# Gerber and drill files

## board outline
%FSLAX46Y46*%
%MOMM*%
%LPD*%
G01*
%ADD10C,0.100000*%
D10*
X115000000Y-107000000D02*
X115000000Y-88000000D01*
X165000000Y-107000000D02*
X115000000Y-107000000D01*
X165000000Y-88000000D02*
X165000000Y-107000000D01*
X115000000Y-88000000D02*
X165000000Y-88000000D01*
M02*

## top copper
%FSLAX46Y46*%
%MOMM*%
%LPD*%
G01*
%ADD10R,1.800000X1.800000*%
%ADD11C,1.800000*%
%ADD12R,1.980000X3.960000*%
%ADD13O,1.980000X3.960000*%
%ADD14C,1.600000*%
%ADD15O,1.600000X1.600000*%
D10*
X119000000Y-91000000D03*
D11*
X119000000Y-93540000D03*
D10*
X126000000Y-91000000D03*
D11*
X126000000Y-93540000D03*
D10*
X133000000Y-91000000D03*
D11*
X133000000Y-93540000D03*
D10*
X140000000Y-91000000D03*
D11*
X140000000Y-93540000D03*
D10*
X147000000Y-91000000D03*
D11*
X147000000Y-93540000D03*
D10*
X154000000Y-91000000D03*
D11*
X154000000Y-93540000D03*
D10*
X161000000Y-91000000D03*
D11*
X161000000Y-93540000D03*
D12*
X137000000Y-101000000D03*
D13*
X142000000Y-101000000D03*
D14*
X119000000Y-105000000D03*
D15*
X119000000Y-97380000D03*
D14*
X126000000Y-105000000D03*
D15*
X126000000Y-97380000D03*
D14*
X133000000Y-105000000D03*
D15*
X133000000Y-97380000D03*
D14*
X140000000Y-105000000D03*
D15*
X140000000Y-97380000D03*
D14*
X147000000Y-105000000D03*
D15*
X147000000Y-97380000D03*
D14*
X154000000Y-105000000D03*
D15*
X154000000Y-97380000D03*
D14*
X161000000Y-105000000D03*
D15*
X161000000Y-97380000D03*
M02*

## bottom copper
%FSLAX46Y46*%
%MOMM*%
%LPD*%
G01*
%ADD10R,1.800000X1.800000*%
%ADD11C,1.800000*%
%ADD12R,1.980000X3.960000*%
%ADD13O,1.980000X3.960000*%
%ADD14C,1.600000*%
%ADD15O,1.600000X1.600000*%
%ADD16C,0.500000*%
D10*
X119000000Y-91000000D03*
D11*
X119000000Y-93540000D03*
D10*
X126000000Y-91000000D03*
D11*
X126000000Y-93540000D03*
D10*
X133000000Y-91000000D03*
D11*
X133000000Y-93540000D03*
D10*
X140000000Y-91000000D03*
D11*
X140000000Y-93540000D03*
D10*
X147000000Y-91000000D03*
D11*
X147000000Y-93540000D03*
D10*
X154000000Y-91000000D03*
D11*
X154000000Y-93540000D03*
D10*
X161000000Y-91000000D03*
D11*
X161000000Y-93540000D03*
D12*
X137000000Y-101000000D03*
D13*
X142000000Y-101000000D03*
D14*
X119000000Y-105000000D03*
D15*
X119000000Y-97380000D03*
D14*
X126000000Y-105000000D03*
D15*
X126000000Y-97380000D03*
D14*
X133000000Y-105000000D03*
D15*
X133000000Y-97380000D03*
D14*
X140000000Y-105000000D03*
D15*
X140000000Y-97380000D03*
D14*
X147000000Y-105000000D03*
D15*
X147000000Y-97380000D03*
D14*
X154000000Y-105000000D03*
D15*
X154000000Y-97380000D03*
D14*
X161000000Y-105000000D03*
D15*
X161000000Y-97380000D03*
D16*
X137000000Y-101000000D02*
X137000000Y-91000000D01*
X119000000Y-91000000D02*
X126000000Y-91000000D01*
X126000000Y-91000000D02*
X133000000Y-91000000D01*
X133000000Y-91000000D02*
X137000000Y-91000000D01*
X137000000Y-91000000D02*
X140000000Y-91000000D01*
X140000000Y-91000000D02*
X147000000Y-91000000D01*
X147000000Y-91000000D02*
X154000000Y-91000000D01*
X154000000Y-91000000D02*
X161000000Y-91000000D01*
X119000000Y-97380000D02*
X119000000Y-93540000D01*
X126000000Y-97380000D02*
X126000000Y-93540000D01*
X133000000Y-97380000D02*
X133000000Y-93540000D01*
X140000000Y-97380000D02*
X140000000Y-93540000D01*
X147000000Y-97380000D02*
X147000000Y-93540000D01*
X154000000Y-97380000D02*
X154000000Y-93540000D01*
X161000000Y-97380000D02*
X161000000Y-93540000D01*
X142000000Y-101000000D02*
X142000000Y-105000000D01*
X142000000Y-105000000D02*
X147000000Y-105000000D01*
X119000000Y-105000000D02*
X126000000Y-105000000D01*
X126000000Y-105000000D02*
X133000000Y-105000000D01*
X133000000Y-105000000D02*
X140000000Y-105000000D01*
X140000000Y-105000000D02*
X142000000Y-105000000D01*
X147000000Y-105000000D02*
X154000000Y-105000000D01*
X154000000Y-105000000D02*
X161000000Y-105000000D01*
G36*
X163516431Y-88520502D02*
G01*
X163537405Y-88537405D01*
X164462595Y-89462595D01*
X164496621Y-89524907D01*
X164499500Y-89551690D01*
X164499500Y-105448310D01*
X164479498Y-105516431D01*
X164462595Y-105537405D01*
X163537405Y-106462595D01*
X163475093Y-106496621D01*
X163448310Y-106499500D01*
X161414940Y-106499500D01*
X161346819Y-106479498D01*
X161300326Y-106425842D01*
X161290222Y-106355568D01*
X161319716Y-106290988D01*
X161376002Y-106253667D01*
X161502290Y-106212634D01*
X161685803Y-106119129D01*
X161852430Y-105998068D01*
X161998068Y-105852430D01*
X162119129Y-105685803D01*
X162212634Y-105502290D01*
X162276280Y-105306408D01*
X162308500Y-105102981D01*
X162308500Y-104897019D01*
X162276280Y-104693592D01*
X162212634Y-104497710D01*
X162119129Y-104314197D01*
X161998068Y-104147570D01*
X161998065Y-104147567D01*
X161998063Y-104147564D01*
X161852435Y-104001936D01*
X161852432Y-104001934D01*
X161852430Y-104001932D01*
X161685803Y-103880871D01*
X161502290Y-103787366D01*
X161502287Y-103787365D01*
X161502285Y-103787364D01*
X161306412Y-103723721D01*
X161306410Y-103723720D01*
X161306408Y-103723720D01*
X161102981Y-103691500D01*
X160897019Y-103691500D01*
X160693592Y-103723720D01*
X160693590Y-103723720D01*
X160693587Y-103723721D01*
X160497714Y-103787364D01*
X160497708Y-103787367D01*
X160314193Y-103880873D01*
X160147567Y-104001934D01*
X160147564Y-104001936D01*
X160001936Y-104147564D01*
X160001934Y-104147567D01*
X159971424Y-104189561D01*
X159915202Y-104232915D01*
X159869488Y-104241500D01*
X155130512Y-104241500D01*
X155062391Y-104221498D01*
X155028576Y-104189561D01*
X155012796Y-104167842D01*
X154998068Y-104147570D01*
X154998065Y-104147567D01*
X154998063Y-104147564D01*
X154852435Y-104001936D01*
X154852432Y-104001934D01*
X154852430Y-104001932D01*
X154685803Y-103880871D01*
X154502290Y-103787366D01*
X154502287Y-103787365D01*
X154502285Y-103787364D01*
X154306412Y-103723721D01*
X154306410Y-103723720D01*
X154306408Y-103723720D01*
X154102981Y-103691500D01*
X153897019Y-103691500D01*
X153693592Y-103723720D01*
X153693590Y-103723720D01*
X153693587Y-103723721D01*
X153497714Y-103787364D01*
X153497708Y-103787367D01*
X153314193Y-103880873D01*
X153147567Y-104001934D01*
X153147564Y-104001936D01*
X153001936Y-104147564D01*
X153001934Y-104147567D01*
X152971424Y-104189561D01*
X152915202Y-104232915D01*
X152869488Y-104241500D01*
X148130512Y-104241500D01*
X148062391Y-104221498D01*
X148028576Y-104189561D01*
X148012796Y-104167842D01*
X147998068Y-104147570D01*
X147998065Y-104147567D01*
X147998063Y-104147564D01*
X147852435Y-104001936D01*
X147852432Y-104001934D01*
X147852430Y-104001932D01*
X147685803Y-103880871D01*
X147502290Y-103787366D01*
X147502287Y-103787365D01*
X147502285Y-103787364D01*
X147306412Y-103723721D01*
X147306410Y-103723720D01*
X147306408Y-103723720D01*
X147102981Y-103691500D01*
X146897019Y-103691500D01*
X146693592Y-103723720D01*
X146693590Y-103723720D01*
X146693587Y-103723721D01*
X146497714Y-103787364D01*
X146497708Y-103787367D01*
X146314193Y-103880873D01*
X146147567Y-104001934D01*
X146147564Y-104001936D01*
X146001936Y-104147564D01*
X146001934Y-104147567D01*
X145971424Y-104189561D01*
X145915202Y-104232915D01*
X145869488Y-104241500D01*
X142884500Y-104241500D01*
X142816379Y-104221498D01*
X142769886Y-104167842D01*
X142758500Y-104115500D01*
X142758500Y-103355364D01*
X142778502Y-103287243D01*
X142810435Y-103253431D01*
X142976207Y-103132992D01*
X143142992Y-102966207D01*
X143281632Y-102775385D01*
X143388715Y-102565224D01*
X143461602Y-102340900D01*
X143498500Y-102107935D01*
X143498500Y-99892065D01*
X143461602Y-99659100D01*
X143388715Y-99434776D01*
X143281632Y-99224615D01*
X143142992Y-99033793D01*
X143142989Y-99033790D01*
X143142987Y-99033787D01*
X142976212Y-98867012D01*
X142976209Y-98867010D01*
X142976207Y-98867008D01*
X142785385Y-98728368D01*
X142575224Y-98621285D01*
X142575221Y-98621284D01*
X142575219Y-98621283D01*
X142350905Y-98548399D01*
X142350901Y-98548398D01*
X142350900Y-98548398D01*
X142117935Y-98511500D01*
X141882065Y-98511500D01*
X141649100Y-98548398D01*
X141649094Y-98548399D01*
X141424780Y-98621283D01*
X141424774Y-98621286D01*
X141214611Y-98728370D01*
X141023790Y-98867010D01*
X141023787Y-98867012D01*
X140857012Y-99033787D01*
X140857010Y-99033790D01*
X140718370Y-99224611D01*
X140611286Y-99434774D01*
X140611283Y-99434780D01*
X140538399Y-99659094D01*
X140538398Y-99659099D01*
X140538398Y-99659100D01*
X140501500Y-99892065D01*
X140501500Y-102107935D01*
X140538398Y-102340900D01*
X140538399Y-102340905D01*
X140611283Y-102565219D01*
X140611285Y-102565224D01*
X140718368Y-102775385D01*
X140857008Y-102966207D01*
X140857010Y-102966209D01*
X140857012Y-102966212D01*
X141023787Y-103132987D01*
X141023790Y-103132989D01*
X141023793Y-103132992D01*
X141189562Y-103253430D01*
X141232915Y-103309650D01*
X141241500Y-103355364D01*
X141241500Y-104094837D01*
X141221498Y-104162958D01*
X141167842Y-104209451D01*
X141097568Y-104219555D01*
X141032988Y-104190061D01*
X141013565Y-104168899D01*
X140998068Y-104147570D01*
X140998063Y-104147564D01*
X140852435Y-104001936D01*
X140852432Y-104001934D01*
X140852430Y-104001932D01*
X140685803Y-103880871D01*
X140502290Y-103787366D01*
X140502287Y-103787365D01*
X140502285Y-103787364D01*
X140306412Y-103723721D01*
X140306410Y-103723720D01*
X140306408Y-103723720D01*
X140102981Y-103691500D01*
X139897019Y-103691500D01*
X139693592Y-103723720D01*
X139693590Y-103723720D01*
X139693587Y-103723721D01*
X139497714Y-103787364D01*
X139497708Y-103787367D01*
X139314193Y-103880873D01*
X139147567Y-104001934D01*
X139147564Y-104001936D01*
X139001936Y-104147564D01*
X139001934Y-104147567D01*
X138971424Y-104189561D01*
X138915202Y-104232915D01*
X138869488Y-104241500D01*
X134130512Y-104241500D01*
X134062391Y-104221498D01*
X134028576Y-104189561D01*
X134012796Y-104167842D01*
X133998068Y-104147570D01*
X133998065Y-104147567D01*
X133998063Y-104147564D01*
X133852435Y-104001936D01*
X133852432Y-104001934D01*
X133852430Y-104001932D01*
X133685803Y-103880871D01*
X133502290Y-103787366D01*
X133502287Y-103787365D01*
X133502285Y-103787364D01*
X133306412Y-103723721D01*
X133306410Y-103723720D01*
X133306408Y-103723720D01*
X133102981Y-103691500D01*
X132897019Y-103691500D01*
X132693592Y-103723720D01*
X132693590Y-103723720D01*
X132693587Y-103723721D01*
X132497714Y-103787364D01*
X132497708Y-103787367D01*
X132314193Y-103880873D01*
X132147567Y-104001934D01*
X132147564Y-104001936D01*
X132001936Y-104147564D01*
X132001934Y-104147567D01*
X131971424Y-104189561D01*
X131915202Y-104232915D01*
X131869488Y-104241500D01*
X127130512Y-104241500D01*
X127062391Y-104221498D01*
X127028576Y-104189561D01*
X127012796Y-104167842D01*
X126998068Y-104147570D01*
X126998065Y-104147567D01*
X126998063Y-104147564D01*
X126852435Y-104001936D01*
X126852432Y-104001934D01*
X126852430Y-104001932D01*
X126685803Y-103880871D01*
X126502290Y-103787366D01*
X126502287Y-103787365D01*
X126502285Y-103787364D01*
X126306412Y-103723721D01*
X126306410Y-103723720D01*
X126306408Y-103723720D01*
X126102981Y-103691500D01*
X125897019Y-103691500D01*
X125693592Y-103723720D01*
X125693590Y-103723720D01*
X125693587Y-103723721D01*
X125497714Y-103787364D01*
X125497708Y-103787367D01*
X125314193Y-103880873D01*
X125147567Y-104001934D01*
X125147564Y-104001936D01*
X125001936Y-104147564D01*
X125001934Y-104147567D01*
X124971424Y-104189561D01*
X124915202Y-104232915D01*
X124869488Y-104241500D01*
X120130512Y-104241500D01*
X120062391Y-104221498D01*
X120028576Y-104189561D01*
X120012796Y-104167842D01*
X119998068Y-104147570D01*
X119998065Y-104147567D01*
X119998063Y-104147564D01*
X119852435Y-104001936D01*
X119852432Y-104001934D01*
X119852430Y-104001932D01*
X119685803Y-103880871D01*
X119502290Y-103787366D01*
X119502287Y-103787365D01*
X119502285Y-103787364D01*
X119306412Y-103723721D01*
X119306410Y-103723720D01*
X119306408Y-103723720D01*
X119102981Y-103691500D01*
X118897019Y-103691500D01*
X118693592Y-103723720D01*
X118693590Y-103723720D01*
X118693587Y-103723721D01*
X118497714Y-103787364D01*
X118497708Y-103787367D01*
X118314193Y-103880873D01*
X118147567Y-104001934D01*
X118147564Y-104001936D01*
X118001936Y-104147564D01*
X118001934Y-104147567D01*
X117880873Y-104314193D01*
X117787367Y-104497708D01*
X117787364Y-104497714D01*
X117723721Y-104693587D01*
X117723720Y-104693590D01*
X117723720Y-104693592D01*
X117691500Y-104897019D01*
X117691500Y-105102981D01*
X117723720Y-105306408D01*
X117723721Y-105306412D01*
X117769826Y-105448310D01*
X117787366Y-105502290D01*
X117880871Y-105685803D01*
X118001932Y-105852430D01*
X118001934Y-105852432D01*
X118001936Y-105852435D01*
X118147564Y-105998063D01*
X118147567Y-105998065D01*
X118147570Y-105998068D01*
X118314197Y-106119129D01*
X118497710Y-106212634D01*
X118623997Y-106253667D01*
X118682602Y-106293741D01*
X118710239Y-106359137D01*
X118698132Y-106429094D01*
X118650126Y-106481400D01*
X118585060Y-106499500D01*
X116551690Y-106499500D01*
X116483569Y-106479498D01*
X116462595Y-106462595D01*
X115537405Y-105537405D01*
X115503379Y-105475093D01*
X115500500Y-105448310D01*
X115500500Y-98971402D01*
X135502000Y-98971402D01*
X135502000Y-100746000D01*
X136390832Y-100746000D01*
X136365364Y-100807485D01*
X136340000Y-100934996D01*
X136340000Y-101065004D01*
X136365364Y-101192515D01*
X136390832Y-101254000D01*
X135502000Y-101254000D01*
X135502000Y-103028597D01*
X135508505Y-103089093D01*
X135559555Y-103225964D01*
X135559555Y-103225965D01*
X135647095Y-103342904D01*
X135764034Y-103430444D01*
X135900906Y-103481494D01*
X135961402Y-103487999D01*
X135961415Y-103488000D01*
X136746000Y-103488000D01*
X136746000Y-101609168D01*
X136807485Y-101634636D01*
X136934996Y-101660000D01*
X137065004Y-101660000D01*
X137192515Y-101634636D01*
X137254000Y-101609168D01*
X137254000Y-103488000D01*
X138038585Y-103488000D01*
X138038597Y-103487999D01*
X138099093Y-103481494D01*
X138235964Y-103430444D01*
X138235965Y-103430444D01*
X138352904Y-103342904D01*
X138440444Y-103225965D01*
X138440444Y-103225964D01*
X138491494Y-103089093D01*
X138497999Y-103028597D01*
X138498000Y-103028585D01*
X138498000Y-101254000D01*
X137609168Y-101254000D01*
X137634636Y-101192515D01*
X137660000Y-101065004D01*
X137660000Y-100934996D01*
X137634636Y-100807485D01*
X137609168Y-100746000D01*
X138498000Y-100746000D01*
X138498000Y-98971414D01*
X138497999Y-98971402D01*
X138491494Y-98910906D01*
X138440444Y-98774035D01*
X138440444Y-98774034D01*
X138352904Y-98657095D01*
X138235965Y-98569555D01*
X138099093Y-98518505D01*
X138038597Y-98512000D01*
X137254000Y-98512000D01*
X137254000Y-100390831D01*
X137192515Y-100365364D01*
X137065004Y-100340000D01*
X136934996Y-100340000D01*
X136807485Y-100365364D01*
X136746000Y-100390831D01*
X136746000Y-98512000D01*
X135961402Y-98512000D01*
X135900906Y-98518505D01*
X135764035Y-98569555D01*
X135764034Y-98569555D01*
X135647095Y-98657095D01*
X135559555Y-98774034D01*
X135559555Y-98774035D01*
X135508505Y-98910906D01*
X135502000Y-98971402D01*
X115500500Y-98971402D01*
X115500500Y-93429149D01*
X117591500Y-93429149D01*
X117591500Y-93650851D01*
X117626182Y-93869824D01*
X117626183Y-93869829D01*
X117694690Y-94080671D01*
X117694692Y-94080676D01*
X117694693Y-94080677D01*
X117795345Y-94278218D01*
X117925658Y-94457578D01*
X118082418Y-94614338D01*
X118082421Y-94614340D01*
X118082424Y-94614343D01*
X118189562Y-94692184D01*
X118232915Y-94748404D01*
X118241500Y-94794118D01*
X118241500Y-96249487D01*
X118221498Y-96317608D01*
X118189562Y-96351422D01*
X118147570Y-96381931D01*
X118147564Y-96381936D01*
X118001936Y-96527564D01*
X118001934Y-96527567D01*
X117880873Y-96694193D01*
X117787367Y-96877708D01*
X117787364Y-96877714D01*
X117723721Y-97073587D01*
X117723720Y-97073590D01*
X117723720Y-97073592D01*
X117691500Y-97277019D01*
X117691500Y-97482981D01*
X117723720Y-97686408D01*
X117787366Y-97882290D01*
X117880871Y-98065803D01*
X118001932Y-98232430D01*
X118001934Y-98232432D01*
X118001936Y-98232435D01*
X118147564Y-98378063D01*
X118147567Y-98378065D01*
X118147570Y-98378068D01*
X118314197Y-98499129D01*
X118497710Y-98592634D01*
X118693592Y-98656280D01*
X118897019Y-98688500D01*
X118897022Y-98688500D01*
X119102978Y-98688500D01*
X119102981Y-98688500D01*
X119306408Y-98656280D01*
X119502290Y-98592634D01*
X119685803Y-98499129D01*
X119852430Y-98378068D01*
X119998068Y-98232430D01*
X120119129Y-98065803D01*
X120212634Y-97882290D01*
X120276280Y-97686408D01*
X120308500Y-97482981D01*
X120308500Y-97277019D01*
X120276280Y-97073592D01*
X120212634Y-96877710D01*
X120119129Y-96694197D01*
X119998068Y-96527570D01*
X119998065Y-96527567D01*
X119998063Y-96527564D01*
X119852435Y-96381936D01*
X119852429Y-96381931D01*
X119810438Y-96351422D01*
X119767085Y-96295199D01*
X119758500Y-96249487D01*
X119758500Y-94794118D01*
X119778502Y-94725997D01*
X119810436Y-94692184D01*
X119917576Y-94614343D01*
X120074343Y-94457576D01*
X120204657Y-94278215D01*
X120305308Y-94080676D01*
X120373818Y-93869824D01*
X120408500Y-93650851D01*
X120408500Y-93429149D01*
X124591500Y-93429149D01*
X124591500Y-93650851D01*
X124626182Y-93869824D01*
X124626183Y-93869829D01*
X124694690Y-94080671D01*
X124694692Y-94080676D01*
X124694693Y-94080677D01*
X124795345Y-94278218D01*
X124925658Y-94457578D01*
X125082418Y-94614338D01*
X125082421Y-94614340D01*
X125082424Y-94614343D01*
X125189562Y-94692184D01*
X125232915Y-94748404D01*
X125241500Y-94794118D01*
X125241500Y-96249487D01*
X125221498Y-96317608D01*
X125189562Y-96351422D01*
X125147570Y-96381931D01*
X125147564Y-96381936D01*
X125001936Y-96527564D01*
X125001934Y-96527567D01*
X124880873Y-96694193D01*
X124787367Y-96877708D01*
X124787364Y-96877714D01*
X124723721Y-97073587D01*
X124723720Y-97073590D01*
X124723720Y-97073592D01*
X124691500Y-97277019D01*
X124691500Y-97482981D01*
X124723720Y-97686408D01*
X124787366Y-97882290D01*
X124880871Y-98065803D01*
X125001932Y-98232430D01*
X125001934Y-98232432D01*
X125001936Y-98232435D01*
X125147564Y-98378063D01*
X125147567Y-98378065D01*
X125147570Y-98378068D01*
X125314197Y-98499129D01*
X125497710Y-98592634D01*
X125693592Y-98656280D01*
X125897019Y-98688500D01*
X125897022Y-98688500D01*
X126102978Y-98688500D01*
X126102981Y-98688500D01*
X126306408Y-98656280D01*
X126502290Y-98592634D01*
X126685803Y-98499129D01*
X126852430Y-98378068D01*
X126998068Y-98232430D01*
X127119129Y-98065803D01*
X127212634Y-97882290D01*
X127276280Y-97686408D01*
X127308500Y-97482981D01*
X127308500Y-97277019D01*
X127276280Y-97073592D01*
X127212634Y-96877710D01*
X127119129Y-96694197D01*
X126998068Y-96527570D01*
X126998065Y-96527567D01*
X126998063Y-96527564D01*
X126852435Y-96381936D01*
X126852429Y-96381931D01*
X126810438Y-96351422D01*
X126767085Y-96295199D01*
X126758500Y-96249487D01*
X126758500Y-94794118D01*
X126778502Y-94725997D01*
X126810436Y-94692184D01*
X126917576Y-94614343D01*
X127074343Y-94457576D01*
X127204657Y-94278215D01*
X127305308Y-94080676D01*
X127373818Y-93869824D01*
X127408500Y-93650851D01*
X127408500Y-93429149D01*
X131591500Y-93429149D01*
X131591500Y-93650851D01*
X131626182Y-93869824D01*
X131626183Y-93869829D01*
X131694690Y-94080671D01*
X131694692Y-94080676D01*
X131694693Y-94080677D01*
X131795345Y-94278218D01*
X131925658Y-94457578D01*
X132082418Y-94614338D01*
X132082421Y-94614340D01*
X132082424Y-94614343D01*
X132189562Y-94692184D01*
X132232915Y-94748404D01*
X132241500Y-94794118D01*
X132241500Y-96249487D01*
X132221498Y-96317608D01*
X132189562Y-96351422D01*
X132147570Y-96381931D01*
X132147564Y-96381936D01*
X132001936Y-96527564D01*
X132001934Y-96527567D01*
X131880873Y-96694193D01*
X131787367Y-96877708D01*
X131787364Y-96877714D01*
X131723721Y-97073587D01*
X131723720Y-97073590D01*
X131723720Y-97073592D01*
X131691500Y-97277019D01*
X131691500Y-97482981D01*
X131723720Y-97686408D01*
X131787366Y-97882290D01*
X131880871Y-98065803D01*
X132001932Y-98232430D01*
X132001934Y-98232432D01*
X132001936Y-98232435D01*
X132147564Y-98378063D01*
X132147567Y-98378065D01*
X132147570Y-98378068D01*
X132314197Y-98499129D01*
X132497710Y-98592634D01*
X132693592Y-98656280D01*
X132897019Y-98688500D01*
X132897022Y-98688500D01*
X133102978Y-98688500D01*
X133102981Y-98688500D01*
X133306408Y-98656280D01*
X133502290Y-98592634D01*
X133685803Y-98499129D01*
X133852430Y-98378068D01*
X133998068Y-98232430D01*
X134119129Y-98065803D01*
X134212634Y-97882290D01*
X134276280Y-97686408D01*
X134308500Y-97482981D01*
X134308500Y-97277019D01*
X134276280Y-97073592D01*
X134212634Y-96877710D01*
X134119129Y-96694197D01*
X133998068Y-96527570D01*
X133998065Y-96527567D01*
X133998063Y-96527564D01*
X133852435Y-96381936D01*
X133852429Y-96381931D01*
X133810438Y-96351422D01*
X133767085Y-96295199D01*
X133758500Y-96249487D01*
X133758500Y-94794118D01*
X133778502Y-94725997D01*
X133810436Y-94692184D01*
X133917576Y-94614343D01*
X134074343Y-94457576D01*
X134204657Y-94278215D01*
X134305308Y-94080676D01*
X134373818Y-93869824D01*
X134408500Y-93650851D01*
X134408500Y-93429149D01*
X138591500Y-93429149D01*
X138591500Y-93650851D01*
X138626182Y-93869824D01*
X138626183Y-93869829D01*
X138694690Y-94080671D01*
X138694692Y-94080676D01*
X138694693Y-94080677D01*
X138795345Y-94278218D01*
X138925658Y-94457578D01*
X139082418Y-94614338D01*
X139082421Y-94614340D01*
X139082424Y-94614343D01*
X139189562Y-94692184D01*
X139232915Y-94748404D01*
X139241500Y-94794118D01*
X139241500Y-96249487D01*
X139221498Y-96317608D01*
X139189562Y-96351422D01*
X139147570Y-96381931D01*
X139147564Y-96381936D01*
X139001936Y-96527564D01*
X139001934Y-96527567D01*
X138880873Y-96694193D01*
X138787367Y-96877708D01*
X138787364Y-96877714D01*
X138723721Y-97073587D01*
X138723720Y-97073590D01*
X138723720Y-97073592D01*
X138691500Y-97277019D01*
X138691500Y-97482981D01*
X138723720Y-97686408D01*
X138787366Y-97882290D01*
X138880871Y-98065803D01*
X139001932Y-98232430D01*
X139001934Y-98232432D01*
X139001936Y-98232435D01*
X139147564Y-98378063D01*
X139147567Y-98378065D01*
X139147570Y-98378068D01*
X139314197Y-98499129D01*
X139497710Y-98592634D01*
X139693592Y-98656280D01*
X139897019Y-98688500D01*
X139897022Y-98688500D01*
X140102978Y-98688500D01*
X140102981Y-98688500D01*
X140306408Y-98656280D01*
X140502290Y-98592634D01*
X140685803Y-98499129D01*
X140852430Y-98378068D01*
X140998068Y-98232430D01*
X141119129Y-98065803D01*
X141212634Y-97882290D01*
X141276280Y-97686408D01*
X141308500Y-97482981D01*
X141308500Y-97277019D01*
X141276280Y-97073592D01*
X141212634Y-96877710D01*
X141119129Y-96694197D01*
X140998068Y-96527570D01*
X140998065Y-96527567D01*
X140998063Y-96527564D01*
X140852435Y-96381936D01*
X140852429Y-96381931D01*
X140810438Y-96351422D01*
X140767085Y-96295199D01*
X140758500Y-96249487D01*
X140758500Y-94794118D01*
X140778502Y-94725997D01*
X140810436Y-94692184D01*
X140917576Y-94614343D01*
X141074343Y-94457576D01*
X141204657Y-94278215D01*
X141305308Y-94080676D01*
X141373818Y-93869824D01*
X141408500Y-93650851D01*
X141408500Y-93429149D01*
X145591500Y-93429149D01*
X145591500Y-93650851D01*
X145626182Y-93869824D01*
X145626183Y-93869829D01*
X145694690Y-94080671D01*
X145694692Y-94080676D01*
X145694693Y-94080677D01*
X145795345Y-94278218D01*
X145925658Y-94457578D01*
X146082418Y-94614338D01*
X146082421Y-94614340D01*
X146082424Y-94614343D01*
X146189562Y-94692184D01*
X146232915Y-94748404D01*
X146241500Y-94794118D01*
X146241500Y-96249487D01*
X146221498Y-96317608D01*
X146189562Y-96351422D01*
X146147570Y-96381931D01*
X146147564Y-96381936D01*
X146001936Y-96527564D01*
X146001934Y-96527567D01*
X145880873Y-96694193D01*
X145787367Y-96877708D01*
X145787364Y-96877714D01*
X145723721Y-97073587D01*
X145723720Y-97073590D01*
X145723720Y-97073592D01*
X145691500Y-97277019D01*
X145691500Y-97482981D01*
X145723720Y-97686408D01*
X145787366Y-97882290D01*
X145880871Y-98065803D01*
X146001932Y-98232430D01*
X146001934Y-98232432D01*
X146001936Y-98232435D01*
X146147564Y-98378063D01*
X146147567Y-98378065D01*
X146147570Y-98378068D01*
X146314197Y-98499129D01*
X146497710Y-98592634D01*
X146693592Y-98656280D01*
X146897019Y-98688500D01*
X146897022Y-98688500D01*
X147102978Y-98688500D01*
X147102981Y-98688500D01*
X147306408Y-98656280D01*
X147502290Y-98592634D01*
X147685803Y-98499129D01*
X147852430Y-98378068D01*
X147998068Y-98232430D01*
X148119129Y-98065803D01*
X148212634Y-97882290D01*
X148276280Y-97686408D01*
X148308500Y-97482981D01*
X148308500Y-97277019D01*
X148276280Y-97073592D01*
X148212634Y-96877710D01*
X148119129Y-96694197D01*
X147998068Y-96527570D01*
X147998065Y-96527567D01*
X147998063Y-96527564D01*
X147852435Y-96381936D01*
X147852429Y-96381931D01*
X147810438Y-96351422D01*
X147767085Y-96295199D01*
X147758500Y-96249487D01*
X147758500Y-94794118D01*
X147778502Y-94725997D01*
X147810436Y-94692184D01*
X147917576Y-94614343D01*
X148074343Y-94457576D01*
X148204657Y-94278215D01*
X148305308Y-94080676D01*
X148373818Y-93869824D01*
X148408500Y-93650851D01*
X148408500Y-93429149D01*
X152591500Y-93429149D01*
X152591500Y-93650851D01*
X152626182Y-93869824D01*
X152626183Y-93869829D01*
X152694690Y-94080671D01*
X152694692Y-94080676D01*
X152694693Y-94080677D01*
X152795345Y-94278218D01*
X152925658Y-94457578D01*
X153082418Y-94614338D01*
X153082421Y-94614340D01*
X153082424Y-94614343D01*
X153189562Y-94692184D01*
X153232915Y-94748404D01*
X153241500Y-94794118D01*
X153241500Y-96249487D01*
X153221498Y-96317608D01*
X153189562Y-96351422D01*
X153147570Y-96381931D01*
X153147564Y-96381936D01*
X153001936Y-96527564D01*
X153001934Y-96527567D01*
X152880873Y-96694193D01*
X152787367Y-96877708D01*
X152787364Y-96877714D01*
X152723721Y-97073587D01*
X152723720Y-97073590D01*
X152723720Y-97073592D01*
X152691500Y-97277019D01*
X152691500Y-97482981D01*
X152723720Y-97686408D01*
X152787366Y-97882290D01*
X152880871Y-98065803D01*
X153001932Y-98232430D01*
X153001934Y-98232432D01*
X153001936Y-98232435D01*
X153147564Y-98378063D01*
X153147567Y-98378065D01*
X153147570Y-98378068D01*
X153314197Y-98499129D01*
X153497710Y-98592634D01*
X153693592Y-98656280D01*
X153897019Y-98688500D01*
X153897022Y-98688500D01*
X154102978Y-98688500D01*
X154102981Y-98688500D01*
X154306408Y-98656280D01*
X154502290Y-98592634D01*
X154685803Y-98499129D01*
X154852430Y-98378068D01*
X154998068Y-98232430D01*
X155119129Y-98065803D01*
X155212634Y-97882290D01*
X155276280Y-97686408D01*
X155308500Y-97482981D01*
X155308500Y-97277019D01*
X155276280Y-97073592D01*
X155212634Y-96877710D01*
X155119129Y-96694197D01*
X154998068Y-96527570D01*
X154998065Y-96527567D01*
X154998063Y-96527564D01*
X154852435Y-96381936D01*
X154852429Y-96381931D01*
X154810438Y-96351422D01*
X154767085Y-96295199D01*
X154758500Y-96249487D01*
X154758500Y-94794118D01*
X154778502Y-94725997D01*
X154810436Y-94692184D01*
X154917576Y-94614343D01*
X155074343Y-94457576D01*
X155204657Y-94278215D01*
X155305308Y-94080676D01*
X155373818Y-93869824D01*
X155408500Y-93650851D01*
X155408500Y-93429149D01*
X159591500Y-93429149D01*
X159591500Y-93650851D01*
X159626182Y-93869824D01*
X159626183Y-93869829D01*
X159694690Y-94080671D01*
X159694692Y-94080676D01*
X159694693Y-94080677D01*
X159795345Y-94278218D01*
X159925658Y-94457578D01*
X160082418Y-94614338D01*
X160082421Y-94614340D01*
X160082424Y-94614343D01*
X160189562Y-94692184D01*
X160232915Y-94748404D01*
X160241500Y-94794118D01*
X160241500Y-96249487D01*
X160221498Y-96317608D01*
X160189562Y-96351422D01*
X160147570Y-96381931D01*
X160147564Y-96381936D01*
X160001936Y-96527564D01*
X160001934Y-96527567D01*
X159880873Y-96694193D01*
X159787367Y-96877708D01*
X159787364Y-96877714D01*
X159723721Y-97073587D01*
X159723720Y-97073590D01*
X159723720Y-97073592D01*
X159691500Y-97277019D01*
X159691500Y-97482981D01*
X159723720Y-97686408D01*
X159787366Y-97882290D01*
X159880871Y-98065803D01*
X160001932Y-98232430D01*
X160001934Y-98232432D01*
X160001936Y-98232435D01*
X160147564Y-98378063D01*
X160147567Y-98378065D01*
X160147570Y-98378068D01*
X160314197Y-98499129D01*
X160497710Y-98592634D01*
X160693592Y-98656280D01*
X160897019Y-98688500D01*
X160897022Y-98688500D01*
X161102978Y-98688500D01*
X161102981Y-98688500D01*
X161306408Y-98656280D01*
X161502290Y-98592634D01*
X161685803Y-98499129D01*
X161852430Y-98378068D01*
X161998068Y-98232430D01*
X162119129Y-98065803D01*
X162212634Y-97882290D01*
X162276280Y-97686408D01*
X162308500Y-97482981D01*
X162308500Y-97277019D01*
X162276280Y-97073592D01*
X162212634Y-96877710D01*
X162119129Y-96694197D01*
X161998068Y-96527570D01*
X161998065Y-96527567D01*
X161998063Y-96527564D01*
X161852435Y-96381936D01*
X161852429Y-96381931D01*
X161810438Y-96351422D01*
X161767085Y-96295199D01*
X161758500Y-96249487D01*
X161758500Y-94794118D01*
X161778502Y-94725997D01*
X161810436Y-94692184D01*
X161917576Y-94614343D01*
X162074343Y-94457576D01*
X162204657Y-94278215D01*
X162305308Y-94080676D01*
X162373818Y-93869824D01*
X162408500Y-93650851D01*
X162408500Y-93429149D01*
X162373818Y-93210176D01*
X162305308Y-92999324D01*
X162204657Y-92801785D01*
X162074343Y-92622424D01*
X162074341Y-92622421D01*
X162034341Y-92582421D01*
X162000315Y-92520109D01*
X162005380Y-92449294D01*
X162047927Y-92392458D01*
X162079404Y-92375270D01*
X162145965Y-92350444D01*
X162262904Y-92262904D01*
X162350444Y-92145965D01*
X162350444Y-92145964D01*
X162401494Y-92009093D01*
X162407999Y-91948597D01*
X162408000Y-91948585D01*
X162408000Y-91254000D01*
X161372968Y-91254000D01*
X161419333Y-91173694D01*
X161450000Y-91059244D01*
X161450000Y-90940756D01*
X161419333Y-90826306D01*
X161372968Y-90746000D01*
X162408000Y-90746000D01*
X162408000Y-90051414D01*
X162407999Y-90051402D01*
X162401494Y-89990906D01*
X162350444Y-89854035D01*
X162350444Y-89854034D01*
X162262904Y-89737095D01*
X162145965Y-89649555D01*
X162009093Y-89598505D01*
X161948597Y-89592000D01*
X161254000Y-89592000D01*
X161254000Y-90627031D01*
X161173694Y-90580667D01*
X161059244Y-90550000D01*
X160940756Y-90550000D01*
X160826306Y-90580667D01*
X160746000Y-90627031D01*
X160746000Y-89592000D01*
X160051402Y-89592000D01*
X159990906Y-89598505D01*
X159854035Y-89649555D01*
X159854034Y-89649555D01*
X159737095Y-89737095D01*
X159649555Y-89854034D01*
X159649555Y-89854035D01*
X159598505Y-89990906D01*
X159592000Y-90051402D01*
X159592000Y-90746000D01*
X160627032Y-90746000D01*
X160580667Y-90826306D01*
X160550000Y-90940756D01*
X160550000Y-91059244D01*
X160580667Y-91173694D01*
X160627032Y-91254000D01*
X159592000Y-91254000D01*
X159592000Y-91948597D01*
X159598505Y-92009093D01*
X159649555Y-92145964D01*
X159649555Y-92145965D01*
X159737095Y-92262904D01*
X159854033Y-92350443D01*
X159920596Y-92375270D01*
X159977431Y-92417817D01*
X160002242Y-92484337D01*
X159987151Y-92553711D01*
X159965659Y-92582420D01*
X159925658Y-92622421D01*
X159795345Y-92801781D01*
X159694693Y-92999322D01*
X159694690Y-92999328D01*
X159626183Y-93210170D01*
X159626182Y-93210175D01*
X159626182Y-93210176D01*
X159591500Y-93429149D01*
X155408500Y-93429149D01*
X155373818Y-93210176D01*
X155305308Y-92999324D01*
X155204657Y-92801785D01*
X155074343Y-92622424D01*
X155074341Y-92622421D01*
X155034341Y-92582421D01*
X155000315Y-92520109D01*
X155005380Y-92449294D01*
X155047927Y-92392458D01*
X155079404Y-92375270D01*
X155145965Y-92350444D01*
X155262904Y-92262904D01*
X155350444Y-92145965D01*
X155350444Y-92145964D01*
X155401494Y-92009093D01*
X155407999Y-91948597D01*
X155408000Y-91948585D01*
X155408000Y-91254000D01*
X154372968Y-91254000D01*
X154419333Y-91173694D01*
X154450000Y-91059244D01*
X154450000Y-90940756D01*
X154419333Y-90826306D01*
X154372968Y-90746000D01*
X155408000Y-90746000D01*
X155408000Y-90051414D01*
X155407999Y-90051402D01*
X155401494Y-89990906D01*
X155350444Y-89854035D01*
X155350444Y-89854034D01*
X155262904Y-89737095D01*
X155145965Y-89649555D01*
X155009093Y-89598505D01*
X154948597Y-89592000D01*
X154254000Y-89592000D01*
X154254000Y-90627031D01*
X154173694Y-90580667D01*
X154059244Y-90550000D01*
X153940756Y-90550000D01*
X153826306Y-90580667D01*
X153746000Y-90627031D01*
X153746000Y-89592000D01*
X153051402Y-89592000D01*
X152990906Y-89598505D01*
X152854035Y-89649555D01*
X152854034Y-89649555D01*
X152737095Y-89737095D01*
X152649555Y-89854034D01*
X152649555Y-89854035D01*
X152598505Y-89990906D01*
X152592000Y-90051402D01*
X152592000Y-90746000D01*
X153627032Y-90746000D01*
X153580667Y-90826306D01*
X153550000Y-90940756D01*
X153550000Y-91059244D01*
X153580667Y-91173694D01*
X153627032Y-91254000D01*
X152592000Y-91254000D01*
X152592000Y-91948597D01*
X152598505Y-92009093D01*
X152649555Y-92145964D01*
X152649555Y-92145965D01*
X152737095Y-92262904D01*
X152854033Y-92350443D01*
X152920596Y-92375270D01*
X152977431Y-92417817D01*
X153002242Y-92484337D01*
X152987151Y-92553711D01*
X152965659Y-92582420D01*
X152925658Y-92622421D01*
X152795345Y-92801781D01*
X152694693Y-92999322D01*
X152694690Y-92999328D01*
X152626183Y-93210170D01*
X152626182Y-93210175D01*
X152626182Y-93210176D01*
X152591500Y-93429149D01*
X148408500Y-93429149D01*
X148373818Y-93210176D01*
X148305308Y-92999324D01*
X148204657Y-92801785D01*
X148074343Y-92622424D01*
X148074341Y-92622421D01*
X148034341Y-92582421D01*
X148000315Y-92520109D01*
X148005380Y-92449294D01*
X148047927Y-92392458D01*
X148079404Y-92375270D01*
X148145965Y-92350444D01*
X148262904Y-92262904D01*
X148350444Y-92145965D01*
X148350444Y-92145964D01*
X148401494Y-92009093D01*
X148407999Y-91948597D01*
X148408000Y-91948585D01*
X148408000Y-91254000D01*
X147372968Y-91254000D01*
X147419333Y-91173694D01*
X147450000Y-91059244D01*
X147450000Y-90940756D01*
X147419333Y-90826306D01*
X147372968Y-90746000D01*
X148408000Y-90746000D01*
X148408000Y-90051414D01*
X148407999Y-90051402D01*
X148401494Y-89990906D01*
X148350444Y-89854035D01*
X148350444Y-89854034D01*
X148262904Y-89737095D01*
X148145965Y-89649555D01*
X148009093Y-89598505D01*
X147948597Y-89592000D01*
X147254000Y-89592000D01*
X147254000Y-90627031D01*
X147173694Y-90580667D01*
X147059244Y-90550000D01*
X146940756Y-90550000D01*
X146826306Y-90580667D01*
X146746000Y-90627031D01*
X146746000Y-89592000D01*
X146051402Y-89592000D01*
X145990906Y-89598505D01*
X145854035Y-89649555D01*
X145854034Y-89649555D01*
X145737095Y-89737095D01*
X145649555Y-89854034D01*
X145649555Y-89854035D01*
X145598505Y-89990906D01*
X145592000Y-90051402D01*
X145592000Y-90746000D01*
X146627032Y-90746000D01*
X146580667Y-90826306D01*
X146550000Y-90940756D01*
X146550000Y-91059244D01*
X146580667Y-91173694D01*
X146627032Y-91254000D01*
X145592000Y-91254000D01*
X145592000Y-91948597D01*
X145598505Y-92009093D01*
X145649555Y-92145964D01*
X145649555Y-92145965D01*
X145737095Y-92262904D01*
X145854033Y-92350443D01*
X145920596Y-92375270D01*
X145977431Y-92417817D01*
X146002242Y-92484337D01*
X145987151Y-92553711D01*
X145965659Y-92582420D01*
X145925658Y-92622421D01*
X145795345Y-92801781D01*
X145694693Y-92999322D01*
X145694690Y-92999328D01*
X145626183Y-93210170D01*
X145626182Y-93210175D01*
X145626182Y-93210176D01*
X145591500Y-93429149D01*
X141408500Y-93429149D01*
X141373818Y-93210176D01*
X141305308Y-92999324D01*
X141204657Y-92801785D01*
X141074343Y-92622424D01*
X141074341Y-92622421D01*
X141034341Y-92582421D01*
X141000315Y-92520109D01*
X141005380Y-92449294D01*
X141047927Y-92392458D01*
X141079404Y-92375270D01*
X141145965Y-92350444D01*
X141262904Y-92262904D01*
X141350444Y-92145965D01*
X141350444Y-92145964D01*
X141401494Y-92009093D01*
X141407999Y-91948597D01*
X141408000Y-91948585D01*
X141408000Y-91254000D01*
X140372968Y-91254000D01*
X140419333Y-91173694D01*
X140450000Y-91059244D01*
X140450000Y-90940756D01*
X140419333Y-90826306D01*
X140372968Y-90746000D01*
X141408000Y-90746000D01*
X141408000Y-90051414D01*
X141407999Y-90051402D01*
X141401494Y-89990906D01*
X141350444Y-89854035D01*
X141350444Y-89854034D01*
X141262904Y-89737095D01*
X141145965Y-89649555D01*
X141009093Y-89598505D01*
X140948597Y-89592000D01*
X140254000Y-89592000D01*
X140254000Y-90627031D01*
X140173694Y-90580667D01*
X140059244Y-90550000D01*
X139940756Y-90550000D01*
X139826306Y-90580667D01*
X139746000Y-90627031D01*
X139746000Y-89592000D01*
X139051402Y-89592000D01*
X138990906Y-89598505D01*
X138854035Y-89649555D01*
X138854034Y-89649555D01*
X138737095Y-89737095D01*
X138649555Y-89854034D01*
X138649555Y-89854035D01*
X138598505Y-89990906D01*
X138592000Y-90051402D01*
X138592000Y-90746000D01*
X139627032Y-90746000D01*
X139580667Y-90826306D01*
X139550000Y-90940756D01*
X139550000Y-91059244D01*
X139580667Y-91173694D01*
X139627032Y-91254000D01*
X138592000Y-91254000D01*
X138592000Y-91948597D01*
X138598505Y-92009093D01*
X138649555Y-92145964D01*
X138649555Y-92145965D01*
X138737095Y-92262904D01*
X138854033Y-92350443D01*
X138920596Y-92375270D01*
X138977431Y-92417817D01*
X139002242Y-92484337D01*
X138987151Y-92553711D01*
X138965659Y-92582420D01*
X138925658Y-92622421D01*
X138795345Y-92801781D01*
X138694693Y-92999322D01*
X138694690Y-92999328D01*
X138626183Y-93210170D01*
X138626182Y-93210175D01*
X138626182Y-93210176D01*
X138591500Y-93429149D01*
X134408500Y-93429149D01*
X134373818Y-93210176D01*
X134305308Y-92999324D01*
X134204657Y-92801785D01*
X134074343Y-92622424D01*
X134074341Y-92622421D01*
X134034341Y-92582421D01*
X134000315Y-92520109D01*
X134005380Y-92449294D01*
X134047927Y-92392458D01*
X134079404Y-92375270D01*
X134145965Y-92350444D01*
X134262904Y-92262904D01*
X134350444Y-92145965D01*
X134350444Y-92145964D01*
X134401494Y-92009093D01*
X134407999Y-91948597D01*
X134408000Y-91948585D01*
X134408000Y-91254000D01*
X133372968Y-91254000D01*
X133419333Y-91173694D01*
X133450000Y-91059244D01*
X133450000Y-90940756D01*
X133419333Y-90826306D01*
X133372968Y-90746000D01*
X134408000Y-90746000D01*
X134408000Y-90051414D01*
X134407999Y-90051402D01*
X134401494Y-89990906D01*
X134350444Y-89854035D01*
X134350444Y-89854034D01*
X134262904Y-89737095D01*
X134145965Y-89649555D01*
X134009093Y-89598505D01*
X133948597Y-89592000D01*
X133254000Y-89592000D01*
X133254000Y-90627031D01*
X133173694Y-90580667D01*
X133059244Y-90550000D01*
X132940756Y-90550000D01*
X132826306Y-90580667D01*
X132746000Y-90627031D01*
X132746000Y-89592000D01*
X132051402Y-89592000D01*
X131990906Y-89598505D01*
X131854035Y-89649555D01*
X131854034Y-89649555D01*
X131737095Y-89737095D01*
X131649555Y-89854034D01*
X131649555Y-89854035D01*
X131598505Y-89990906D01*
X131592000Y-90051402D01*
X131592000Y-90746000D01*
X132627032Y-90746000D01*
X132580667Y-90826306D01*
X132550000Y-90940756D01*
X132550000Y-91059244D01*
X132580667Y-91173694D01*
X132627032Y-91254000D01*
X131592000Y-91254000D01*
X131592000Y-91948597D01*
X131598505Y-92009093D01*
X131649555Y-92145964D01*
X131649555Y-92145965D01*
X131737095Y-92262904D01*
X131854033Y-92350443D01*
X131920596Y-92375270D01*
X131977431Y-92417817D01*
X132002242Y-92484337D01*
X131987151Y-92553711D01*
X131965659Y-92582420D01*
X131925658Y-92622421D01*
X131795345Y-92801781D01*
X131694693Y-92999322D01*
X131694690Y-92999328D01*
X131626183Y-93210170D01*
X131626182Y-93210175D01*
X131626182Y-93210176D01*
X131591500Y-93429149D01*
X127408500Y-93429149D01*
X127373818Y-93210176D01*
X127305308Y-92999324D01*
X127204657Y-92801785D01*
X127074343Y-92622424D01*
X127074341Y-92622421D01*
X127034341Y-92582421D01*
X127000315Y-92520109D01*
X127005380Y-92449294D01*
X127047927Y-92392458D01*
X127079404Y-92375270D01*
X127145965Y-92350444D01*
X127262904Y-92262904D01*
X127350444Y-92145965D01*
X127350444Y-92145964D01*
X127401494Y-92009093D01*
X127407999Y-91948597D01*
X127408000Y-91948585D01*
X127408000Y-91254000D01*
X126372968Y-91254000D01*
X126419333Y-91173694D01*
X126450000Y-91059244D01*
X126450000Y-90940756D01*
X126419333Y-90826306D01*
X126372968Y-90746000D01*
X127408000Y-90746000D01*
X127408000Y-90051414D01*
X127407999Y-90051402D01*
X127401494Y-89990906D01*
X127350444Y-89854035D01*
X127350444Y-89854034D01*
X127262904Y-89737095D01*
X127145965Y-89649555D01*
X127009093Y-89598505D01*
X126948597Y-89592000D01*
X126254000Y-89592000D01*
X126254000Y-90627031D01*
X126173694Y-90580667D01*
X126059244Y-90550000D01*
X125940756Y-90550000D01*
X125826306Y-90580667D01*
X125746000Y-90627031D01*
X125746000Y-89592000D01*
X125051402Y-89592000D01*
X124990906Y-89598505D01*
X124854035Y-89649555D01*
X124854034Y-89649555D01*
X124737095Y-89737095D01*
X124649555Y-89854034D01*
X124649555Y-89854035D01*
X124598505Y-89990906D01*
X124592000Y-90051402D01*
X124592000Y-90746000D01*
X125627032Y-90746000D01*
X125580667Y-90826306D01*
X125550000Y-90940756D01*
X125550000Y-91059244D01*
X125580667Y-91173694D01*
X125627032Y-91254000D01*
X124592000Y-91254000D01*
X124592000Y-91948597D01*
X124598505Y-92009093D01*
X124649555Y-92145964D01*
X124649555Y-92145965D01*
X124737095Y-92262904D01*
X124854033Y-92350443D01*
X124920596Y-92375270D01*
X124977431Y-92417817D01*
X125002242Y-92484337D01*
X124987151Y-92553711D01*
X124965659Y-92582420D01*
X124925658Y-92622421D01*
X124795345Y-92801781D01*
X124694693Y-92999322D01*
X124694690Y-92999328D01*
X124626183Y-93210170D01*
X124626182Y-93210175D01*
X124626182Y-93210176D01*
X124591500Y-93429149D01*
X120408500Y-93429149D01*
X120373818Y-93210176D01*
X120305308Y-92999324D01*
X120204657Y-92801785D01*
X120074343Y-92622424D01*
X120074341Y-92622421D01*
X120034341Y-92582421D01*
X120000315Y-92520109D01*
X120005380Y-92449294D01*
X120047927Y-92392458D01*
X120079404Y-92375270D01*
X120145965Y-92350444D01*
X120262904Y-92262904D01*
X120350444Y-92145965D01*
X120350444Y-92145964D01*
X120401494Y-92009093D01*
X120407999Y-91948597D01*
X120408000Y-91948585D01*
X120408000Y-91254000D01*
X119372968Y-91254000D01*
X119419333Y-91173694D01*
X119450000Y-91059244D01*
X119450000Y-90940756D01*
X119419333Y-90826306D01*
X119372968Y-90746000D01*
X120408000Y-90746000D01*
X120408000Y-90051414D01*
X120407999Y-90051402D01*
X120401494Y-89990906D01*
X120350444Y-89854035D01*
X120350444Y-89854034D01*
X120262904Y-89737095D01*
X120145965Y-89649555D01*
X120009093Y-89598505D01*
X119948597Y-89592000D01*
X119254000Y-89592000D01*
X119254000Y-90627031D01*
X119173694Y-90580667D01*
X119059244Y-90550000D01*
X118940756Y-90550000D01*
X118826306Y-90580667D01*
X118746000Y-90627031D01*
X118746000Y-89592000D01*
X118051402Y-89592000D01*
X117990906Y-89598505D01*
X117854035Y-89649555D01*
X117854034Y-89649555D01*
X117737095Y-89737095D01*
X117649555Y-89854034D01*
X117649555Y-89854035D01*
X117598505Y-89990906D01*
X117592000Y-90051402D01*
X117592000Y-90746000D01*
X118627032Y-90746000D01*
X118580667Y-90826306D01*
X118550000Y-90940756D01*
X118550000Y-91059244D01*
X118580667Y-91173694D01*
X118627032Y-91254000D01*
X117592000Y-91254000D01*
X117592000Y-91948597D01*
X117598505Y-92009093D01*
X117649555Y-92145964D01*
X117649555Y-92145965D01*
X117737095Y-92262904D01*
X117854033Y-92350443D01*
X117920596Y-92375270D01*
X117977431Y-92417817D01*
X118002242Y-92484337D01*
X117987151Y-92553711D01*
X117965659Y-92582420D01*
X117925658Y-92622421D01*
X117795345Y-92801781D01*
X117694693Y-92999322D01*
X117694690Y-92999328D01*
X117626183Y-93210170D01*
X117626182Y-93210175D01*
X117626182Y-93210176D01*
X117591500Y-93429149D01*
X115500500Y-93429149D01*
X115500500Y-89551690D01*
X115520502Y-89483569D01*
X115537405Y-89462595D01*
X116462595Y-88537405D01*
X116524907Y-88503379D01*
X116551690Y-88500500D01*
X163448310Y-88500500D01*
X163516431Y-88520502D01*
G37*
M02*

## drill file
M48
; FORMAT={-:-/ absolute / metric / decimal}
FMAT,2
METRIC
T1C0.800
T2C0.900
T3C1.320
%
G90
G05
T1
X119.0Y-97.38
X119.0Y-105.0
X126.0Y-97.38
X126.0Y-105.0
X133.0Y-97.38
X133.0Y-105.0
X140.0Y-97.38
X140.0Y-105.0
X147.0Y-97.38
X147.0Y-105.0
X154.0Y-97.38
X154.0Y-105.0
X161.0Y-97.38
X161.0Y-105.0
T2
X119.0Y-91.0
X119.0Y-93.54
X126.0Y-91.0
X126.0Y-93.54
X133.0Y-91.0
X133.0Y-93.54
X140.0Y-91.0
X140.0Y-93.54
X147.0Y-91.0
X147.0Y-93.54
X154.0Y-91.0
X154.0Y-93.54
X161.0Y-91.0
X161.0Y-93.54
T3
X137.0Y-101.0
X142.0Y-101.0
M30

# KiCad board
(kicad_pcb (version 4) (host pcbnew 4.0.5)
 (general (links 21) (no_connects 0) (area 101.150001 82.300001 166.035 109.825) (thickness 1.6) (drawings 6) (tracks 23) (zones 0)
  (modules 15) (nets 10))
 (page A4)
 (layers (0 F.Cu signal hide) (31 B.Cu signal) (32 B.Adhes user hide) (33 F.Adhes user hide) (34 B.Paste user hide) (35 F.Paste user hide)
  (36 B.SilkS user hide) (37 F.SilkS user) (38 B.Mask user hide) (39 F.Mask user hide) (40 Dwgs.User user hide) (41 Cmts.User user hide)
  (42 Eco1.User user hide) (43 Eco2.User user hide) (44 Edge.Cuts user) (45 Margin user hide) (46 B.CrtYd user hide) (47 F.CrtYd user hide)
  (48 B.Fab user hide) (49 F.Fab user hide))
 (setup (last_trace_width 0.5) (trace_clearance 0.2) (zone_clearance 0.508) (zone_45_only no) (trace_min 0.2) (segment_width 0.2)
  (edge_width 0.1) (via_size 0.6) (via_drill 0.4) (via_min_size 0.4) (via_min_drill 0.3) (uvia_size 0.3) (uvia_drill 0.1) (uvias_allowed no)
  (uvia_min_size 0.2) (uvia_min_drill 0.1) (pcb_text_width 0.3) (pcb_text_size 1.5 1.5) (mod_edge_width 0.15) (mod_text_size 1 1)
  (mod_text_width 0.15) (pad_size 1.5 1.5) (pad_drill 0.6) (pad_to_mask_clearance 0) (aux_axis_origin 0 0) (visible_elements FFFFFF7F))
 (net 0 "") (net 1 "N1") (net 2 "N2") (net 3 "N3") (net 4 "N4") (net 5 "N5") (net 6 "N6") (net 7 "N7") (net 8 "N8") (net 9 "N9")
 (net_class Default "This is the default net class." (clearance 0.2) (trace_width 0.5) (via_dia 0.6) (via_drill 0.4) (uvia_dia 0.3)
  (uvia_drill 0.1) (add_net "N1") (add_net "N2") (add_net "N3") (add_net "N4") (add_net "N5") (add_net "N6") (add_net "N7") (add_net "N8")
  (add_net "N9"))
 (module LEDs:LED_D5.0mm (layer F.Cu) (at 119 91 270)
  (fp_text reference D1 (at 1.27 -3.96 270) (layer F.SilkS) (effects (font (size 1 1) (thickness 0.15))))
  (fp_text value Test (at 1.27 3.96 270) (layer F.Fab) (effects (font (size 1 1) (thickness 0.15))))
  (pad 1 thru_hole rect (at 0 0 270) (size 1.8 1.8) (drill 0.9) (layers *.Cu *.Mask) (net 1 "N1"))
  (pad 2 thru_hole circle (at 2.54 0 270) (size 1.8 1.8) (drill 0.9) (layers *.Cu *.Mask) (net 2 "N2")))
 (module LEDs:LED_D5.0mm (layer F.Cu) (at 126 91 270)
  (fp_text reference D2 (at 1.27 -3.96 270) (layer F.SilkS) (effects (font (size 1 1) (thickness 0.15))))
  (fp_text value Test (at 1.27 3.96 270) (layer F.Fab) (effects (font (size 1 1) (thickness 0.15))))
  (pad 1 thru_hole rect (at 0 0 270) (size 1.8 1.8) (drill 0.9) (layers *.Cu *.Mask) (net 1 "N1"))
  (pad 2 thru_hole circle (at 2.54 0 270) (size 1.8 1.8) (drill 0.9) (layers *.Cu *.Mask) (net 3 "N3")))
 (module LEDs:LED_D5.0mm (layer F.Cu) (at 133 91 270)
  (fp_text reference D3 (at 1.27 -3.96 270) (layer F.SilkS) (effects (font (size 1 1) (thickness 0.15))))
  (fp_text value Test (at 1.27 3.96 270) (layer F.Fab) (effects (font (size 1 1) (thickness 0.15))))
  (pad 1 thru_hole rect (at 0 0 270) (size 1.8 1.8) (drill 0.9) (layers *.Cu *.Mask) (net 1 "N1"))
  (pad 2 thru_hole circle (at 2.54 0 270) (size 1.8 1.8) (drill 0.9) (layers *.Cu *.Mask) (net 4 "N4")))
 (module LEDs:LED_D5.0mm (layer F.Cu) (at 140 91 270)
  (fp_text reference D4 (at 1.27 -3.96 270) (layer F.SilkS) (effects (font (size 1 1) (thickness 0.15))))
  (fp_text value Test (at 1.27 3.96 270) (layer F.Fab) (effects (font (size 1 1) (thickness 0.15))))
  (pad 1 thru_hole rect (at 0 0 270) (size 1.8 1.8) (drill 0.9) (layers *.Cu *.Mask) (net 1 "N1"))
  (pad 2 thru_hole circle (at 2.54 0 270) (size 1.8 1.8) (drill 0.9) (layers *.Cu *.Mask) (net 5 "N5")))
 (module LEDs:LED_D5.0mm (layer F.Cu) (at 147 91 270)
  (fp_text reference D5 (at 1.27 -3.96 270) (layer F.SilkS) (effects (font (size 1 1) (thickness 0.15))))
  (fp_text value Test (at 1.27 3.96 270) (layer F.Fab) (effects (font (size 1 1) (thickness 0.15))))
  (pad 1 thru_hole rect (at 0 0 270) (size 1.8 1.8) (drill 0.9) (layers *.Cu *.Mask) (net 1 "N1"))
  (pad 2 thru_hole circle (at 2.54 0 270) (size 1.8 1.8) (drill 0.9) (layers *.Cu *.Mask) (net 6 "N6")))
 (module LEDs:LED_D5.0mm (layer F.Cu) (at 154 91 270)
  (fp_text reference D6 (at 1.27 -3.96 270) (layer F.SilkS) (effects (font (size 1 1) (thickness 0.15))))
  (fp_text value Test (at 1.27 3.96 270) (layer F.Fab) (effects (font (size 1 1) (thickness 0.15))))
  (pad 1 thru_hole rect (at 0 0 270) (size 1.8 1.8) (drill 0.9) (layers *.Cu *.Mask) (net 1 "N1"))
  (pad 2 thru_hole circle (at 2.54 0 270) (size 1.8 1.8) (drill 0.9) (layers *.Cu *.Mask) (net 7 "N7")))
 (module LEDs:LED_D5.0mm (layer F.Cu) (at 161 91 270)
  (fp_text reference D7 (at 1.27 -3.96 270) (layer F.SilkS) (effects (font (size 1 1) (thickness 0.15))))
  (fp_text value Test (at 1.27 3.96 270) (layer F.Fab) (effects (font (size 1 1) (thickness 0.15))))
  (pad 1 thru_hole rect (at 0 0 270) (size 1.8 1.8) (drill 0.9) (layers *.Cu *.Mask) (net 1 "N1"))
  (pad 2 thru_hole circle (at 2.54 0 270) (size 1.8 1.8) (drill 0.9) (layers *.Cu *.Mask) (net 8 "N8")))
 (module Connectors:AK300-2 (layer F.Cu) (at 137 101)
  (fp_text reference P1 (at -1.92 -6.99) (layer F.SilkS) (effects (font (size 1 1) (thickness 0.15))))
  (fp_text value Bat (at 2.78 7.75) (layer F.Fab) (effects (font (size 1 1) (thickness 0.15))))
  (pad 1 thru_hole rect (at 0 0) (size 1.98 3.96) (drill 1.32) (layers *.Cu F.Paste F.Mask) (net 1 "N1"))
  (pad 2 thru_hole oval (at 5 0) (size 1.98 3.96) (drill 1.32) (layers *.Cu F.Paste F.Mask) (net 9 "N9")))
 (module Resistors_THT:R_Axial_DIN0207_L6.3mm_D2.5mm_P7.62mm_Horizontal (layer F.Cu) (at 119 105 90)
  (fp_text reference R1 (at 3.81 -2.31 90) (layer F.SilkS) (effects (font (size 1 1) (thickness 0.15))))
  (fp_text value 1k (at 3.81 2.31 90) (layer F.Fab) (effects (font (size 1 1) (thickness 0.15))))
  (pad 1 thru_hole circle (at 0 0 90) (size 1.6 1.6) (drill 0.8) (layers *.Cu *.Mask) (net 9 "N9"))
  (pad 2 thru_hole oval (at 7.62 0 90) (size 1.6 1.6) (drill 0.8) (layers *.Cu *.Mask) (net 2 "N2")))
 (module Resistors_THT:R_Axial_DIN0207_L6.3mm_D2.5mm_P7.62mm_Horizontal (layer F.Cu) (at 126 105 90)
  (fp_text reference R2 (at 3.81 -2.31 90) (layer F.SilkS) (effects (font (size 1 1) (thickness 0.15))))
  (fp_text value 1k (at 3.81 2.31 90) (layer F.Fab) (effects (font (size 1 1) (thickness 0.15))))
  (pad 1 thru_hole circle (at 0 0 90) (size 1.6 1.6) (drill 0.8) (layers *.Cu *.Mask) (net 9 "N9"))
  (pad 2 thru_hole oval (at 7.62 0 90) (size 1.6 1.6) (drill 0.8) (layers *.Cu *.Mask) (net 3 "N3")))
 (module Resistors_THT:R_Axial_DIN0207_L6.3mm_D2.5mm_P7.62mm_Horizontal (layer F.Cu) (at 133 105 90)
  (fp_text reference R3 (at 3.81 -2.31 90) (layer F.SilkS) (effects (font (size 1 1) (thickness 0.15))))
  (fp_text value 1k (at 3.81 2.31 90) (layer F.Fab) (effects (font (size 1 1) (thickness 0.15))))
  (pad 1 thru_hole circle (at 0 0 90) (size 1.6 1.6) (drill 0.8) (layers *.Cu *.Mask) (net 9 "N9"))
  (pad 2 thru_hole oval (at 7.62 0 90) (size 1.6 1.6) (drill 0.8) (layers *.Cu *.Mask) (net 4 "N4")))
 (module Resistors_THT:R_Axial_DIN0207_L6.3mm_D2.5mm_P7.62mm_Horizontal (layer F.Cu) (at 140 105 90)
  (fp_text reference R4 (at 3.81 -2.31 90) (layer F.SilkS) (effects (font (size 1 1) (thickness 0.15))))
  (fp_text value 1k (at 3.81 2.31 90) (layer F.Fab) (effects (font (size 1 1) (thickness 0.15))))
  (pad 1 thru_hole circle (at 0 0 90) (size 1.6 1.6) (drill 0.8) (layers *.Cu *.Mask) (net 9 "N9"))
  (pad 2 thru_hole oval (at 7.62 0 90) (size 1.6 1.6) (drill 0.8) (layers *.Cu *.Mask) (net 5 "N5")))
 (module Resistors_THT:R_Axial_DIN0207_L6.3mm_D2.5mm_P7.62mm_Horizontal (layer F.Cu) (at 147 105 90)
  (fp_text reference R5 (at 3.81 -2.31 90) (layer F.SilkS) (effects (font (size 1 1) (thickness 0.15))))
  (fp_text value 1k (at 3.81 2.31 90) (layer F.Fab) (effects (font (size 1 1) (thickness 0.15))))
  (pad 1 thru_hole circle (at 0 0 90) (size 1.6 1.6) (drill 0.8) (layers *.Cu *.Mask) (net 9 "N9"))
  (pad 2 thru_hole oval (at 7.62 0 90) (size 1.6 1.6) (drill 0.8) (layers *.Cu *.Mask) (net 6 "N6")))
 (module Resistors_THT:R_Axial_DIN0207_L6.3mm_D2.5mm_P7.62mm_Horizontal (layer F.Cu) (at 154 105 90)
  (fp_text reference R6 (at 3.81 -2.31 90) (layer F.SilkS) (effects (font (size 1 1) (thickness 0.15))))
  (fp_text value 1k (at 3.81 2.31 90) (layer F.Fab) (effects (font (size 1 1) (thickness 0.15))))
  (pad 1 thru_hole circle (at 0 0 90) (size 1.6 1.6) (drill 0.8) (layers *.Cu *.Mask) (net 9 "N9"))
  (pad 2 thru_hole oval (at 7.62 0 90) (size 1.6 1.6) (drill 0.8) (layers *.Cu *.Mask) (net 7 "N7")))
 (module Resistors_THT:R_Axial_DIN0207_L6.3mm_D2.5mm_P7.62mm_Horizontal (layer F.Cu) (at 161 105 90)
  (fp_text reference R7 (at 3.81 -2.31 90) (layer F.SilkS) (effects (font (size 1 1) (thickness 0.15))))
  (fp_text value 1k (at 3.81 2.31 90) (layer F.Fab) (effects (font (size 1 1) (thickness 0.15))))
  (pad 1 thru_hole circle (at 0 0 90) (size 1.6 1.6) (drill 0.8) (layers *.Cu *.Mask) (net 9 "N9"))
  (pad 2 thru_hole oval (at 7.62 0 90) (size 1.6 1.6) (drill 0.8) (layers *.Cu *.Mask) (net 8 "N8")))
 (gr_line (start 115 107) (end 115 88) (angle 90) (layer Edge.Cuts) (width 0.1))
 (gr_line (start 165 107) (end 115 107) (angle 90) (layer Edge.Cuts) (width 0.1))
 (gr_line (start 165 88) (end 165 107) (angle 90) (layer Edge.Cuts) (width 0.1))
 (gr_line (start 115 88) (end 165 88) (angle 90) (layer Edge.Cuts) (width 0.1))
 (segment (start 137 101) (end 137 91) (width 0.5) (layer B.Cu) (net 1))
 (segment (start 119 91) (end 126 91) (width 0.5) (layer B.Cu) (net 1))
 (segment (start 126 91) (end 133 91) (width 0.5) (layer B.Cu) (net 1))
 (segment (start 133 91) (end 137 91) (width 0.5) (layer B.Cu) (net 1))
 (segment (start 137 91) (end 140 91) (width 0.5) (layer B.Cu) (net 1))
 (segment (start 140 91) (end 147 91) (width 0.5) (layer B.Cu) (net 1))
 (segment (start 147 91) (end 154 91) (width 0.5) (layer B.Cu) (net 1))
 (segment (start 154 91) (end 161 91) (width 0.5) (layer B.Cu) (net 1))
 (segment (start 119 97.38) (end 119 93.54) (width 0.5) (layer B.Cu) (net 2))
 (segment (start 126 97.38) (end 126 93.54) (width 0.5) (layer B.Cu) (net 3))
 (segment (start 133 97.38) (end 133 93.54) (width 0.5) (layer B.Cu) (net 4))
 (segment (start 140 97.38) (end 140 93.54) (width 0.5) (layer B.Cu) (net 5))
 (segment (start 147 97.38) (end 147 93.54) (width 0.5) (layer B.Cu) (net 6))
 (segment (start 154 97.38) (end 154 93.54) (width 0.5) (layer B.Cu) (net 7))
 (segment (start 161 97.38) (end 161 93.54) (width 0.5) (layer B.Cu) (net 8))
 (segment (start 142 101) (end 142 105) (width 0.5) (layer B.Cu) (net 9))
 (segment (start 142 105) (end 147 105) (width 0.5) (layer B.Cu) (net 9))
 (segment (start 119 105) (end 126 105) (width 0.5) (layer B.Cu) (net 9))
 (segment (start 126 105) (end 133 105) (width 0.5) (layer B.Cu) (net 9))
 (segment (start 133 105) (end 140 105) (width 0.5) (layer B.Cu) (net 9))
 (segment (start 140 105) (end 142 105) (width 0.5) (layer B.Cu) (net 9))
 (segment (start 147 105) (end 154 105) (width 0.5) (layer B.Cu) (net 9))
 (segment (start 154 105) (end 161 105) (width 0.5) (layer B.Cu) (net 9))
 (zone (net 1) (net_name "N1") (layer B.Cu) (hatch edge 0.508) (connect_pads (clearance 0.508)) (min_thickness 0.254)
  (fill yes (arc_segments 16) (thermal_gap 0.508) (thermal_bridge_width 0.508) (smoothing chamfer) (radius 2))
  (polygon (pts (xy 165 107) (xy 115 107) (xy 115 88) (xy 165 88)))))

